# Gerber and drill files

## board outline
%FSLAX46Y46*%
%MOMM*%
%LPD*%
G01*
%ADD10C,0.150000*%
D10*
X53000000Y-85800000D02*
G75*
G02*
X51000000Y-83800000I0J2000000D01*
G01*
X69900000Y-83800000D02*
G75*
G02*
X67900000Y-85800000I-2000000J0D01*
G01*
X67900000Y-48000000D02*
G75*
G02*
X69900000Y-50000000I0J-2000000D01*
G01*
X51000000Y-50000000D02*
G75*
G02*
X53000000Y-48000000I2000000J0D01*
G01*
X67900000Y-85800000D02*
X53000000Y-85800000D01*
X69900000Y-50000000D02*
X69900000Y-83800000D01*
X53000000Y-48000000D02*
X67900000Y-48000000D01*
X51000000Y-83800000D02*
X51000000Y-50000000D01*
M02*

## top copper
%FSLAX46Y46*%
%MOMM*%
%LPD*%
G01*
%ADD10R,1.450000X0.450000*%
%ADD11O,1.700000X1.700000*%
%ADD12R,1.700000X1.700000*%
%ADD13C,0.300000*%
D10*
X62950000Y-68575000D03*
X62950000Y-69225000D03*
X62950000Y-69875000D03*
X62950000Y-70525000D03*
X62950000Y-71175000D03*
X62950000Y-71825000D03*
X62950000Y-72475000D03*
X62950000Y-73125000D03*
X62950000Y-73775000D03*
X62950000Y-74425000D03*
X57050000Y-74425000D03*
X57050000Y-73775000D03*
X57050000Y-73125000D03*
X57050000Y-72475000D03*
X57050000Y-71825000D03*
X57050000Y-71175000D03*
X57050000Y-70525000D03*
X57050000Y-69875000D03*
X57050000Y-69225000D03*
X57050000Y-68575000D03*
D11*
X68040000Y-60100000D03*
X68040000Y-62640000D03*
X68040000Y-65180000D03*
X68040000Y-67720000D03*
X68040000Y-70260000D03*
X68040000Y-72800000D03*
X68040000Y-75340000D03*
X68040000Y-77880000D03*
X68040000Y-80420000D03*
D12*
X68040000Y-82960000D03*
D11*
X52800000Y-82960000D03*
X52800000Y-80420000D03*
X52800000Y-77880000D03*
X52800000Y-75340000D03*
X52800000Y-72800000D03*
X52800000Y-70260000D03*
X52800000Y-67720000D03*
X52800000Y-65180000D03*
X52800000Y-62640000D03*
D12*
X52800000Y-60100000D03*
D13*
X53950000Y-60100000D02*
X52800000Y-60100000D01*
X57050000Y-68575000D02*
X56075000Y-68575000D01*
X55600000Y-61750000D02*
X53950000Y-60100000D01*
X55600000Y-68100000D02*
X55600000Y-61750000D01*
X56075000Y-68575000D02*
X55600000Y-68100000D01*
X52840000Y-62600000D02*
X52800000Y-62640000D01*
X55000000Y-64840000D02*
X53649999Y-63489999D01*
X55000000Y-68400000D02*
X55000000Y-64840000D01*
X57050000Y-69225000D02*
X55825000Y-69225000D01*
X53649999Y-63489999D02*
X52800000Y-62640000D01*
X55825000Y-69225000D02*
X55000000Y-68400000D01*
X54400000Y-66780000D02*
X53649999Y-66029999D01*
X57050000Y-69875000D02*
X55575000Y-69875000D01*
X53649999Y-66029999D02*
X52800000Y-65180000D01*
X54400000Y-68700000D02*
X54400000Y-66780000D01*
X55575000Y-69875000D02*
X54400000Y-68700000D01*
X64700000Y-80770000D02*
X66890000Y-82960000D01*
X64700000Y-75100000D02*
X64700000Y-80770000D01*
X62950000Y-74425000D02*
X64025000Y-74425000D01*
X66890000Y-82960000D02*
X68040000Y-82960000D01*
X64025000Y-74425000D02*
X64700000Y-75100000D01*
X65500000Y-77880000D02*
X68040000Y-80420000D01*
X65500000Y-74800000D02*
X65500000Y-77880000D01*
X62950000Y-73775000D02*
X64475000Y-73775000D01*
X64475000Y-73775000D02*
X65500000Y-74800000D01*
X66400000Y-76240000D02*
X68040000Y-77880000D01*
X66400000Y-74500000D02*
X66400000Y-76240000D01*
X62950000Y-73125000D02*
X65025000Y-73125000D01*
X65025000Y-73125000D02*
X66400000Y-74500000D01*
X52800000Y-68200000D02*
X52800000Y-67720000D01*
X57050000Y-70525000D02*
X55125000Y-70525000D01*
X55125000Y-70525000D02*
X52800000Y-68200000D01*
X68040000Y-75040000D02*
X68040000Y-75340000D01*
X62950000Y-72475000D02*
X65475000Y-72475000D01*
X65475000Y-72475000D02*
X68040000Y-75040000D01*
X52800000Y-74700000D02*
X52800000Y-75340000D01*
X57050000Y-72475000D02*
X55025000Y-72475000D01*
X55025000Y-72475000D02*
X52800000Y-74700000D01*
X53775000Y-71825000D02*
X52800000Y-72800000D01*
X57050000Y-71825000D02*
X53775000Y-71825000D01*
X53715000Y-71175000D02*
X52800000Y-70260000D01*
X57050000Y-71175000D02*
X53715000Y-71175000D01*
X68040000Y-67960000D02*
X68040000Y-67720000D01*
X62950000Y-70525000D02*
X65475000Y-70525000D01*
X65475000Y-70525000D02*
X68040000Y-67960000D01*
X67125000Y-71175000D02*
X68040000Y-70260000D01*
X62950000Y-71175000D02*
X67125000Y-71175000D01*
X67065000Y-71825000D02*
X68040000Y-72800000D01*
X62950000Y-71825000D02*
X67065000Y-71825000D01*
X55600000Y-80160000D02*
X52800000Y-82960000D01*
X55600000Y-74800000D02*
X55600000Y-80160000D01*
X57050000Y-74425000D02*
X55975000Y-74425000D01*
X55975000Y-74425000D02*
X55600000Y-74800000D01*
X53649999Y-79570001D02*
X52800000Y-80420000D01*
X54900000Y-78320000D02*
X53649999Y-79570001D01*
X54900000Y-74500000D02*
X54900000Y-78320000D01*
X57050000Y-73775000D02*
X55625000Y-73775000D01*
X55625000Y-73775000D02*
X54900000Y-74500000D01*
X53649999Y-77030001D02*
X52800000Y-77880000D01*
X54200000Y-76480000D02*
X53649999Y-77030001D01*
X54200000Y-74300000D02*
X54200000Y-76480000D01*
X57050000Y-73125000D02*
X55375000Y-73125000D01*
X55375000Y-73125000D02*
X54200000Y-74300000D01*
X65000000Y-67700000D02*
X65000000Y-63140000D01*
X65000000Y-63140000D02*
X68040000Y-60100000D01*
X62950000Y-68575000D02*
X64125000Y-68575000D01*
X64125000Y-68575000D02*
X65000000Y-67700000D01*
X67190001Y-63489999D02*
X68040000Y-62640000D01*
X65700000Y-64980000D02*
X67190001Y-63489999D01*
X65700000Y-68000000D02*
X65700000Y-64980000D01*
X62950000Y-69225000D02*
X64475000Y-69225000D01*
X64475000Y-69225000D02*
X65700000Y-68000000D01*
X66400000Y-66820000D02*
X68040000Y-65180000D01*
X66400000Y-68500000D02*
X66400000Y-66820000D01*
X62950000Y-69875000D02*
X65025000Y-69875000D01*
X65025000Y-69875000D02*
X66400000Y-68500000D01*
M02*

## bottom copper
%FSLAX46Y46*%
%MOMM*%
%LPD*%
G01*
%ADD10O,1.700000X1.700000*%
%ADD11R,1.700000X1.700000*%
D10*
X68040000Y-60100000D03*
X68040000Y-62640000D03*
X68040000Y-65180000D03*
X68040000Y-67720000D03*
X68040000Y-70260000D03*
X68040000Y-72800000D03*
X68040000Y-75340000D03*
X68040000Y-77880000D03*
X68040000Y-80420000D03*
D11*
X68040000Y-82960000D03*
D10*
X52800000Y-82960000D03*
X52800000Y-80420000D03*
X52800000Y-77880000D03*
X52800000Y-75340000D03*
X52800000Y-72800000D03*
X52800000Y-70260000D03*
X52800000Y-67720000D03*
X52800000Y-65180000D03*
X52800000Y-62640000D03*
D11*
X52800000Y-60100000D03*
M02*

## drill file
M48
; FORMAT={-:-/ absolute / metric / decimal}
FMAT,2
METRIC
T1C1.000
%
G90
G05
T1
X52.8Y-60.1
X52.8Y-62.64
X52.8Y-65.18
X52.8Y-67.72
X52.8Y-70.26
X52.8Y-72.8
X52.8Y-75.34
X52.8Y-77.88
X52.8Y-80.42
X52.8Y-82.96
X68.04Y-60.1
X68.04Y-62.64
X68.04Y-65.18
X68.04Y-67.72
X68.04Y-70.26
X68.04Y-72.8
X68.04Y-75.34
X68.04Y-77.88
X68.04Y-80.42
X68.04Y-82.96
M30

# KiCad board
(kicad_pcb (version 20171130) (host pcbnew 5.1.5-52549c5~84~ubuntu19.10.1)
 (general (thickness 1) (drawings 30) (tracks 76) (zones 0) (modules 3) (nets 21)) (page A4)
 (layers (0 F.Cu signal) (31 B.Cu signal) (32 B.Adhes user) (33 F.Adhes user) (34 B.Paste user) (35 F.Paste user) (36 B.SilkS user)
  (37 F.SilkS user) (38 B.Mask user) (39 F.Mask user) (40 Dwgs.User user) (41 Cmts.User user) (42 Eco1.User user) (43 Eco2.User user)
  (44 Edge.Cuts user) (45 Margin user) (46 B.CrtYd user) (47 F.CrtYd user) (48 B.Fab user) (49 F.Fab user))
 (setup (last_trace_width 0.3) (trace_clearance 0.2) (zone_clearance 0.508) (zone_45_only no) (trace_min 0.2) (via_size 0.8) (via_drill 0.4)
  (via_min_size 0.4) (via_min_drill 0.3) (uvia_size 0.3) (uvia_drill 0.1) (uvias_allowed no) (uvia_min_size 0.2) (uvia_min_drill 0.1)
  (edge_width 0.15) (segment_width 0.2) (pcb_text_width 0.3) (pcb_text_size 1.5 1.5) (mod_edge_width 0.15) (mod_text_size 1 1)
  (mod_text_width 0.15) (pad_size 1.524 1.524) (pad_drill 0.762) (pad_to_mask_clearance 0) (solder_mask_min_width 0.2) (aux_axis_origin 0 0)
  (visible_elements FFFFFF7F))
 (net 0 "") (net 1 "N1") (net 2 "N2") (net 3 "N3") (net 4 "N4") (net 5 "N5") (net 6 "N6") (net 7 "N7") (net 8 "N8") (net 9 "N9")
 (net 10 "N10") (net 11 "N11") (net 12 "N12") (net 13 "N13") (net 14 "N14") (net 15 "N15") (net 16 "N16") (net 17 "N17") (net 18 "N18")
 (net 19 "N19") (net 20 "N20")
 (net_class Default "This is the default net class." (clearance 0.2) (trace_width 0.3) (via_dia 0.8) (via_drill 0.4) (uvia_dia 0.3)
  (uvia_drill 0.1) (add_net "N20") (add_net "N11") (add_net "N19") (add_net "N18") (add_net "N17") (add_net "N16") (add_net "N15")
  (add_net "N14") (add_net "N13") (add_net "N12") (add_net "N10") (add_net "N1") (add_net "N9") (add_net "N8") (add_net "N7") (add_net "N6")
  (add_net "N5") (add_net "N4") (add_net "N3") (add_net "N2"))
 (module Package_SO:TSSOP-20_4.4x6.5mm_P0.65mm (layer F.Cu) (at 60 71.5)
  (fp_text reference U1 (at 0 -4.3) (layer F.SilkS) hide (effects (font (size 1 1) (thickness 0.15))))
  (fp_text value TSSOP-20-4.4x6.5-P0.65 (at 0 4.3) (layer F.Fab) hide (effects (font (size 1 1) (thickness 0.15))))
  (pad 20 smd rect (at 2.95 -2.925) (size 1.45 0.45) (layers F.Cu F.Paste F.Mask) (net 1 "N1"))
  (pad 19 smd rect (at 2.95 -2.275) (size 1.45 0.45) (layers F.Cu F.Paste F.Mask) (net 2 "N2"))
  (pad 18 smd rect (at 2.95 -1.625) (size 1.45 0.45) (layers F.Cu F.Paste F.Mask) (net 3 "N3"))
  (pad 17 smd rect (at 2.95 -0.975) (size 1.45 0.45) (layers F.Cu F.Paste F.Mask) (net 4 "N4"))
  (pad 16 smd rect (at 2.95 -0.325) (size 1.45 0.45) (layers F.Cu F.Paste F.Mask) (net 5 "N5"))
  (pad 15 smd rect (at 2.95 0.325) (size 1.45 0.45) (layers F.Cu F.Paste F.Mask) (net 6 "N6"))
  (pad 14 smd rect (at 2.95 0.975) (size 1.45 0.45) (layers F.Cu F.Paste F.Mask) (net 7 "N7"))
  (pad 13 smd rect (at 2.95 1.625) (size 1.45 0.45) (layers F.Cu F.Paste F.Mask) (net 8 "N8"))
  (pad 12 smd rect (at 2.95 2.275) (size 1.45 0.45) (layers F.Cu F.Paste F.Mask) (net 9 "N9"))
  (pad 11 smd rect (at 2.95 2.925) (size 1.45 0.45) (layers F.Cu F.Paste F.Mask) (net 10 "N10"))
  (pad 10 smd rect (at -2.95 2.925) (size 1.45 0.45) (layers F.Cu F.Paste F.Mask) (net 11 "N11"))
  (pad 9 smd rect (at -2.95 2.275) (size 1.45 0.45) (layers F.Cu F.Paste F.Mask) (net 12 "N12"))
  (pad 8 smd rect (at -2.95 1.625) (size 1.45 0.45) (layers F.Cu F.Paste F.Mask) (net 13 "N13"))
  (pad 7 smd rect (at -2.95 0.975) (size 1.45 0.45) (layers F.Cu F.Paste F.Mask) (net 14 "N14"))
  (pad 6 smd rect (at -2.95 0.325) (size 1.45 0.45) (layers F.Cu F.Paste F.Mask) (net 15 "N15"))
  (pad 5 smd rect (at -2.95 -0.325) (size 1.45 0.45) (layers F.Cu F.Paste F.Mask) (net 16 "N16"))
  (pad 4 smd rect (at -2.95 -0.975) (size 1.45 0.45) (layers F.Cu F.Paste F.Mask) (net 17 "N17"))
  (pad 3 smd rect (at -2.95 -1.625) (size 1.45 0.45) (layers F.Cu F.Paste F.Mask) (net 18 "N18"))
  (pad 2 smd rect (at -2.95 -2.275) (size 1.45 0.45) (layers F.Cu F.Paste F.Mask) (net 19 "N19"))
  (pad 1 smd rect (at -2.95 -2.925) (size 1.45 0.45) (layers F.Cu F.Paste F.Mask) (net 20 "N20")))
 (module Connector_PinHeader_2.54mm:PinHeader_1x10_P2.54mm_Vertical (layer F.Cu) (at 68.04 82.96 180)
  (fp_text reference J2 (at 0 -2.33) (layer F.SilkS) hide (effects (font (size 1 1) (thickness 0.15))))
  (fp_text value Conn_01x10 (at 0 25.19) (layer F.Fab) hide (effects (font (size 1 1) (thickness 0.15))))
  (pad 10 thru_hole oval (at 0 22.86 180) (size 1.7 1.7) (drill 1) (layers *.Cu *.Mask) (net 1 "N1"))
  (pad 9 thru_hole oval (at 0 20.32 180) (size 1.7 1.7) (drill 1) (layers *.Cu *.Mask) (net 2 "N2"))
  (pad 8 thru_hole oval (at 0 17.78 180) (size 1.7 1.7) (drill 1) (layers *.Cu *.Mask) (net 3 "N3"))
  (pad 7 thru_hole oval (at 0 15.24 180) (size 1.7 1.7) (drill 1) (layers *.Cu *.Mask) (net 4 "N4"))
  (pad 6 thru_hole oval (at 0 12.7 180) (size 1.7 1.7) (drill 1) (layers *.Cu *.Mask) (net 5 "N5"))
  (pad 5 thru_hole oval (at 0 10.16 180) (size 1.7 1.7) (drill 1) (layers *.Cu *.Mask) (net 6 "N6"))
  (pad 4 thru_hole oval (at 0 7.62 180) (size 1.7 1.7) (drill 1) (layers *.Cu *.Mask) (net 7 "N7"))
  (pad 3 thru_hole oval (at 0 5.08 180) (size 1.7 1.7) (drill 1) (layers *.Cu *.Mask) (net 8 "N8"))
  (pad 2 thru_hole oval (at 0 2.54 180) (size 1.7 1.7) (drill 1) (layers *.Cu *.Mask) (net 9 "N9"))
  (pad 1 thru_hole rect (at 0 0 180) (size 1.7 1.7) (drill 1) (layers *.Cu *.Mask) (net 10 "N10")))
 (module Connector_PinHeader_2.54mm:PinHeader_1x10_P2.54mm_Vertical (layer F.Cu) (at 52.8 60.1)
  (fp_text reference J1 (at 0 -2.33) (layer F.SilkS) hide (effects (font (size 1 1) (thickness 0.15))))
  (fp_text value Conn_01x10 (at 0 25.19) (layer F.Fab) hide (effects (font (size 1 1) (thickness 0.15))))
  (pad 10 thru_hole oval (at 0 22.86) (size 1.7 1.7) (drill 1) (layers *.Cu *.Mask) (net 11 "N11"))
  (pad 9 thru_hole oval (at 0 20.32) (size 1.7 1.7) (drill 1) (layers *.Cu *.Mask) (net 12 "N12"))
  (pad 8 thru_hole oval (at 0 17.78) (size 1.7 1.7) (drill 1) (layers *.Cu *.Mask) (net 13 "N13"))
  (pad 7 thru_hole oval (at 0 15.24) (size 1.7 1.7) (drill 1) (layers *.Cu *.Mask) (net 14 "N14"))
  (pad 6 thru_hole oval (at 0 12.7) (size 1.7 1.7) (drill 1) (layers *.Cu *.Mask) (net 15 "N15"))
  (pad 5 thru_hole oval (at 0 10.16) (size 1.7 1.7) (drill 1) (layers *.Cu *.Mask) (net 16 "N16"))
  (pad 4 thru_hole oval (at 0 7.62) (size 1.7 1.7) (drill 1) (layers *.Cu *.Mask) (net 17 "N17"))
  (pad 3 thru_hole oval (at 0 5.08) (size 1.7 1.7) (drill 1) (layers *.Cu *.Mask) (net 18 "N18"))
  (pad 2 thru_hole oval (at 0 2.54) (size 1.7 1.7) (drill 1) (layers *.Cu *.Mask) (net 19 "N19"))
  (pad 1 thru_hole rect (at 0 0) (size 1.7 1.7) (drill 1) (layers *.Cu *.Mask) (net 20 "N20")))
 (gr_arc (start 53 83.8) (end 51 83.8) (angle -90) (layer Edge.Cuts) (width 0.15))
 (gr_arc (start 67.9 83.8) (end 67.9 85.8) (angle -90) (layer Edge.Cuts) (width 0.15))
 (gr_arc (start 67.9 50) (end 69.9 50) (angle -90) (layer Edge.Cuts) (width 0.15))
 (gr_arc (start 53 50) (end 53 48) (angle -90) (layer Edge.Cuts) (width 0.15))
 (gr_line (start 67.9 85.8) (end 53 85.8) (layer Edge.Cuts) (width 0.15))
 (gr_line (start 69.9 50) (end 69.9 83.8) (layer Edge.Cuts) (width 0.15))
 (gr_line (start 53 48) (end 67.9 48) (layer Edge.Cuts) (width 0.15))
 (gr_line (start 51 83.8) (end 51 50) (layer Edge.Cuts) (width 0.15))
 (segment (start 53.95 60.1) (end 52.8 60.1) (width 0.3) (layer F.Cu) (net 20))
 (segment (start 57.05 68.575) (end 56.075 68.575) (width 0.3) (layer F.Cu) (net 20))
 (segment (start 55.6 61.75) (end 53.95 60.1) (width 0.3) (layer F.Cu) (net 20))
 (segment (start 55.6 68.1) (end 55.6 61.75) (width 0.3) (layer F.Cu) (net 20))
 (segment (start 56.075 68.575) (end 55.6 68.1) (width 0.3) (layer F.Cu) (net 20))
 (segment (start 52.84 62.6) (end 52.8 62.64) (width 0.3) (layer F.Cu) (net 19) (status 30))
 (segment (start 55 64.84) (end 53.649999 63.489999) (width 0.3) (layer F.Cu) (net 19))
 (segment (start 55 68.4) (end 55 64.84) (width 0.3) (layer F.Cu) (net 19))
 (segment (start 57.05 69.225) (end 55.825 69.225) (width 0.3) (layer F.Cu) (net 19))
 (segment (start 53.649999 63.489999) (end 52.8 62.64) (width 0.3) (layer F.Cu) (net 19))
 (segment (start 55.825 69.225) (end 55 68.4) (width 0.3) (layer F.Cu) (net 19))
 (segment (start 54.4 66.78) (end 53.649999 66.029999) (width 0.3) (layer F.Cu) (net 18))
 (segment (start 57.05 69.875) (end 55.575 69.875) (width 0.3) (layer F.Cu) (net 18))
 (segment (start 53.649999 66.029999) (end 52.8 65.18) (width 0.3) (layer F.Cu) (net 18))
 (segment (start 54.4 68.7) (end 54.4 66.78) (width 0.3) (layer F.Cu) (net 18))
 (segment (start 55.575 69.875) (end 54.4 68.7) (width 0.3) (layer F.Cu) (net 18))
 (segment (start 64.7 80.77) (end 66.89 82.96) (width 0.3) (layer F.Cu) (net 10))
 (segment (start 64.7 75.1) (end 64.7 80.77) (width 0.3) (layer F.Cu) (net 10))
 (segment (start 62.95 74.425) (end 64.025 74.425) (width 0.3) (layer F.Cu) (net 10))
 (segment (start 66.89 82.96) (end 68.04 82.96) (width 0.3) (layer F.Cu) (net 10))
 (segment (start 64.025 74.425) (end 64.7 75.1) (width 0.3) (layer F.Cu) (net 10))
 (segment (start 65.5 77.88) (end 68.04 80.42) (width 0.3) (layer F.Cu) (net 9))
 (segment (start 65.5 74.8) (end 65.5 77.88) (width 0.3) (layer F.Cu) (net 9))
 (segment (start 62.95 73.775) (end 64.475 73.775) (width 0.3) (layer F.Cu) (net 9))
 (segment (start 64.475 73.775) (end 65.5 74.8) (width 0.3) (layer F.Cu) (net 9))
 (segment (start 66.4 76.24) (end 68.04 77.88) (width 0.3) (layer F.Cu) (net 8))
 (segment (start 66.4 74.5) (end 66.4 76.24) (width 0.3) (layer F.Cu) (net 8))
 (segment (start 62.95 73.125) (end 65.025 73.125) (width 0.3) (layer F.Cu) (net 8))
 (segment (start 65.025 73.125) (end 66.4 74.5) (width 0.3) (layer F.Cu) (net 8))
 (segment (start 52.8 68.2) (end 52.8 67.72) (width 0.3) (layer F.Cu) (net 17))
 (segment (start 57.05 70.525) (end 55.125 70.525) (width 0.3) (layer F.Cu) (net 17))
 (segment (start 55.125 70.525) (end 52.8 68.2) (width 0.3) (layer F.Cu) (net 17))
 (segment (start 68.04 75.04) (end 68.04 75.34) (width 0.3) (layer F.Cu) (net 7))
 (segment (start 62.95 72.475) (end 65.475 72.475) (width 0.3) (layer F.Cu) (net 7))
 (segment (start 65.475 72.475) (end 68.04 75.04) (width 0.3) (layer F.Cu) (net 7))
 (segment (start 52.8 74.7) (end 52.8 75.34) (width 0.3) (layer F.Cu) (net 14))
 (segment (start 57.05 72.475) (end 55.025 72.475) (width 0.3) (layer F.Cu) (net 14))
 (segment (start 55.025 72.475) (end 52.8 74.7) (width 0.3) (layer F.Cu) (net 14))
 (segment (start 53.775 71.825) (end 52.8 72.8) (width 0.3) (layer F.Cu) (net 15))
 (segment (start 57.05 71.825) (end 53.775 71.825) (width 0.3) (layer F.Cu) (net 15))
 (segment (start 53.715 71.175) (end 52.8 70.26) (width 0.3) (layer F.Cu) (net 16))
 (segment (start 57.05 71.175) (end 53.715 71.175) (width 0.3) (layer F.Cu) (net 16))
 (segment (start 68.04 67.96) (end 68.04 67.72) (width 0.3) (layer F.Cu) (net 4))
 (segment (start 62.95 70.525) (end 65.475 70.525) (width 0.3) (layer F.Cu) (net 4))
 (segment (start 65.475 70.525) (end 68.04 67.96) (width 0.3) (layer F.Cu) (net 4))
 (segment (start 67.125 71.175) (end 68.04 70.26) (width 0.3) (layer F.Cu) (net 5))
 (segment (start 62.95 71.175) (end 67.125 71.175) (width 0.3) (layer F.Cu) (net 5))
 (segment (start 67.065 71.825) (end 68.04 72.8) (width 0.3) (layer F.Cu) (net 6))
 (segment (start 62.95 71.825) (end 67.065 71.825) (width 0.3) (layer F.Cu) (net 6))
 (segment (start 55.6 80.16) (end 52.8 82.96) (width 0.3) (layer F.Cu) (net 11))
 (segment (start 55.6 74.8) (end 55.6 80.16) (width 0.3) (layer F.Cu) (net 11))
 (segment (start 57.05 74.425) (end 55.975 74.425) (width 0.3) (layer F.Cu) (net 11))
 (segment (start 55.975 74.425) (end 55.6 74.8) (width 0.3) (layer F.Cu) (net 11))
 (segment (start 53.649999 79.570001) (end 52.8 80.42) (width 0.3) (layer F.Cu) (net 12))
 (segment (start 54.9 78.32) (end 53.649999 79.570001) (width 0.3) (layer F.Cu) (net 12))
 (segment (start 54.9 74.5) (end 54.9 78.32) (width 0.3) (layer F.Cu) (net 12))
 (segment (start 57.05 73.775) (end 55.625 73.775) (width 0.3) (layer F.Cu) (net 12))
 (segment (start 55.625 73.775) (end 54.9 74.5) (width 0.3) (layer F.Cu) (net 12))
 (segment (start 53.649999 77.030001) (end 52.8 77.88) (width 0.3) (layer F.Cu) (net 13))
 (segment (start 54.2 76.48) (end 53.649999 77.030001) (width 0.3) (layer F.Cu) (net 13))
 (segment (start 54.2 74.3) (end 54.2 76.48) (width 0.3) (layer F.Cu) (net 13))
 (segment (start 57.05 73.125) (end 55.375 73.125) (width 0.3) (layer F.Cu) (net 13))
 (segment (start 55.375 73.125) (end 54.2 74.3) (width 0.3) (layer F.Cu) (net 13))
 (segment (start 65 67.7) (end 65 63.14) (width 0.3) (layer F.Cu) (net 1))
 (segment (start 65 63.14) (end 68.04 60.1) (width 0.3) (layer F.Cu) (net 1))
 (segment (start 62.95 68.575) (end 64.125 68.575) (width 0.3) (layer F.Cu) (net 1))
 (segment (start 64.125 68.575) (end 65 67.7) (width 0.3) (layer F.Cu) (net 1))
 (segment (start 67.190001 63.489999) (end 68.04 62.64) (width 0.3) (layer F.Cu) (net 2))
 (segment (start 65.7 64.98) (end 67.190001 63.489999) (width 0.3) (layer F.Cu) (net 2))
 (segment (start 65.7 68) (end 65.7 64.98) (width 0.3) (layer F.Cu) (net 2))
 (segment (start 62.95 69.225) (end 64.475 69.225) (width 0.3) (layer F.Cu) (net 2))
 (segment (start 64.475 69.225) (end 65.7 68) (width 0.3) (layer F.Cu) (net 2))
 (segment (start 66.4 66.82) (end 68.04 65.18) (width 0.3) (layer F.Cu) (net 3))
 (segment (start 66.4 68.5) (end 66.4 66.82) (width 0.3) (layer F.Cu) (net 3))
 (segment (start 62.95 69.875) (end 65.025 69.875) (width 0.3) (layer F.Cu) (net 3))
 (segment (start 65.025 69.875) (end 66.4 68.5) (width 0.3) (layer F.Cu) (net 3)))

